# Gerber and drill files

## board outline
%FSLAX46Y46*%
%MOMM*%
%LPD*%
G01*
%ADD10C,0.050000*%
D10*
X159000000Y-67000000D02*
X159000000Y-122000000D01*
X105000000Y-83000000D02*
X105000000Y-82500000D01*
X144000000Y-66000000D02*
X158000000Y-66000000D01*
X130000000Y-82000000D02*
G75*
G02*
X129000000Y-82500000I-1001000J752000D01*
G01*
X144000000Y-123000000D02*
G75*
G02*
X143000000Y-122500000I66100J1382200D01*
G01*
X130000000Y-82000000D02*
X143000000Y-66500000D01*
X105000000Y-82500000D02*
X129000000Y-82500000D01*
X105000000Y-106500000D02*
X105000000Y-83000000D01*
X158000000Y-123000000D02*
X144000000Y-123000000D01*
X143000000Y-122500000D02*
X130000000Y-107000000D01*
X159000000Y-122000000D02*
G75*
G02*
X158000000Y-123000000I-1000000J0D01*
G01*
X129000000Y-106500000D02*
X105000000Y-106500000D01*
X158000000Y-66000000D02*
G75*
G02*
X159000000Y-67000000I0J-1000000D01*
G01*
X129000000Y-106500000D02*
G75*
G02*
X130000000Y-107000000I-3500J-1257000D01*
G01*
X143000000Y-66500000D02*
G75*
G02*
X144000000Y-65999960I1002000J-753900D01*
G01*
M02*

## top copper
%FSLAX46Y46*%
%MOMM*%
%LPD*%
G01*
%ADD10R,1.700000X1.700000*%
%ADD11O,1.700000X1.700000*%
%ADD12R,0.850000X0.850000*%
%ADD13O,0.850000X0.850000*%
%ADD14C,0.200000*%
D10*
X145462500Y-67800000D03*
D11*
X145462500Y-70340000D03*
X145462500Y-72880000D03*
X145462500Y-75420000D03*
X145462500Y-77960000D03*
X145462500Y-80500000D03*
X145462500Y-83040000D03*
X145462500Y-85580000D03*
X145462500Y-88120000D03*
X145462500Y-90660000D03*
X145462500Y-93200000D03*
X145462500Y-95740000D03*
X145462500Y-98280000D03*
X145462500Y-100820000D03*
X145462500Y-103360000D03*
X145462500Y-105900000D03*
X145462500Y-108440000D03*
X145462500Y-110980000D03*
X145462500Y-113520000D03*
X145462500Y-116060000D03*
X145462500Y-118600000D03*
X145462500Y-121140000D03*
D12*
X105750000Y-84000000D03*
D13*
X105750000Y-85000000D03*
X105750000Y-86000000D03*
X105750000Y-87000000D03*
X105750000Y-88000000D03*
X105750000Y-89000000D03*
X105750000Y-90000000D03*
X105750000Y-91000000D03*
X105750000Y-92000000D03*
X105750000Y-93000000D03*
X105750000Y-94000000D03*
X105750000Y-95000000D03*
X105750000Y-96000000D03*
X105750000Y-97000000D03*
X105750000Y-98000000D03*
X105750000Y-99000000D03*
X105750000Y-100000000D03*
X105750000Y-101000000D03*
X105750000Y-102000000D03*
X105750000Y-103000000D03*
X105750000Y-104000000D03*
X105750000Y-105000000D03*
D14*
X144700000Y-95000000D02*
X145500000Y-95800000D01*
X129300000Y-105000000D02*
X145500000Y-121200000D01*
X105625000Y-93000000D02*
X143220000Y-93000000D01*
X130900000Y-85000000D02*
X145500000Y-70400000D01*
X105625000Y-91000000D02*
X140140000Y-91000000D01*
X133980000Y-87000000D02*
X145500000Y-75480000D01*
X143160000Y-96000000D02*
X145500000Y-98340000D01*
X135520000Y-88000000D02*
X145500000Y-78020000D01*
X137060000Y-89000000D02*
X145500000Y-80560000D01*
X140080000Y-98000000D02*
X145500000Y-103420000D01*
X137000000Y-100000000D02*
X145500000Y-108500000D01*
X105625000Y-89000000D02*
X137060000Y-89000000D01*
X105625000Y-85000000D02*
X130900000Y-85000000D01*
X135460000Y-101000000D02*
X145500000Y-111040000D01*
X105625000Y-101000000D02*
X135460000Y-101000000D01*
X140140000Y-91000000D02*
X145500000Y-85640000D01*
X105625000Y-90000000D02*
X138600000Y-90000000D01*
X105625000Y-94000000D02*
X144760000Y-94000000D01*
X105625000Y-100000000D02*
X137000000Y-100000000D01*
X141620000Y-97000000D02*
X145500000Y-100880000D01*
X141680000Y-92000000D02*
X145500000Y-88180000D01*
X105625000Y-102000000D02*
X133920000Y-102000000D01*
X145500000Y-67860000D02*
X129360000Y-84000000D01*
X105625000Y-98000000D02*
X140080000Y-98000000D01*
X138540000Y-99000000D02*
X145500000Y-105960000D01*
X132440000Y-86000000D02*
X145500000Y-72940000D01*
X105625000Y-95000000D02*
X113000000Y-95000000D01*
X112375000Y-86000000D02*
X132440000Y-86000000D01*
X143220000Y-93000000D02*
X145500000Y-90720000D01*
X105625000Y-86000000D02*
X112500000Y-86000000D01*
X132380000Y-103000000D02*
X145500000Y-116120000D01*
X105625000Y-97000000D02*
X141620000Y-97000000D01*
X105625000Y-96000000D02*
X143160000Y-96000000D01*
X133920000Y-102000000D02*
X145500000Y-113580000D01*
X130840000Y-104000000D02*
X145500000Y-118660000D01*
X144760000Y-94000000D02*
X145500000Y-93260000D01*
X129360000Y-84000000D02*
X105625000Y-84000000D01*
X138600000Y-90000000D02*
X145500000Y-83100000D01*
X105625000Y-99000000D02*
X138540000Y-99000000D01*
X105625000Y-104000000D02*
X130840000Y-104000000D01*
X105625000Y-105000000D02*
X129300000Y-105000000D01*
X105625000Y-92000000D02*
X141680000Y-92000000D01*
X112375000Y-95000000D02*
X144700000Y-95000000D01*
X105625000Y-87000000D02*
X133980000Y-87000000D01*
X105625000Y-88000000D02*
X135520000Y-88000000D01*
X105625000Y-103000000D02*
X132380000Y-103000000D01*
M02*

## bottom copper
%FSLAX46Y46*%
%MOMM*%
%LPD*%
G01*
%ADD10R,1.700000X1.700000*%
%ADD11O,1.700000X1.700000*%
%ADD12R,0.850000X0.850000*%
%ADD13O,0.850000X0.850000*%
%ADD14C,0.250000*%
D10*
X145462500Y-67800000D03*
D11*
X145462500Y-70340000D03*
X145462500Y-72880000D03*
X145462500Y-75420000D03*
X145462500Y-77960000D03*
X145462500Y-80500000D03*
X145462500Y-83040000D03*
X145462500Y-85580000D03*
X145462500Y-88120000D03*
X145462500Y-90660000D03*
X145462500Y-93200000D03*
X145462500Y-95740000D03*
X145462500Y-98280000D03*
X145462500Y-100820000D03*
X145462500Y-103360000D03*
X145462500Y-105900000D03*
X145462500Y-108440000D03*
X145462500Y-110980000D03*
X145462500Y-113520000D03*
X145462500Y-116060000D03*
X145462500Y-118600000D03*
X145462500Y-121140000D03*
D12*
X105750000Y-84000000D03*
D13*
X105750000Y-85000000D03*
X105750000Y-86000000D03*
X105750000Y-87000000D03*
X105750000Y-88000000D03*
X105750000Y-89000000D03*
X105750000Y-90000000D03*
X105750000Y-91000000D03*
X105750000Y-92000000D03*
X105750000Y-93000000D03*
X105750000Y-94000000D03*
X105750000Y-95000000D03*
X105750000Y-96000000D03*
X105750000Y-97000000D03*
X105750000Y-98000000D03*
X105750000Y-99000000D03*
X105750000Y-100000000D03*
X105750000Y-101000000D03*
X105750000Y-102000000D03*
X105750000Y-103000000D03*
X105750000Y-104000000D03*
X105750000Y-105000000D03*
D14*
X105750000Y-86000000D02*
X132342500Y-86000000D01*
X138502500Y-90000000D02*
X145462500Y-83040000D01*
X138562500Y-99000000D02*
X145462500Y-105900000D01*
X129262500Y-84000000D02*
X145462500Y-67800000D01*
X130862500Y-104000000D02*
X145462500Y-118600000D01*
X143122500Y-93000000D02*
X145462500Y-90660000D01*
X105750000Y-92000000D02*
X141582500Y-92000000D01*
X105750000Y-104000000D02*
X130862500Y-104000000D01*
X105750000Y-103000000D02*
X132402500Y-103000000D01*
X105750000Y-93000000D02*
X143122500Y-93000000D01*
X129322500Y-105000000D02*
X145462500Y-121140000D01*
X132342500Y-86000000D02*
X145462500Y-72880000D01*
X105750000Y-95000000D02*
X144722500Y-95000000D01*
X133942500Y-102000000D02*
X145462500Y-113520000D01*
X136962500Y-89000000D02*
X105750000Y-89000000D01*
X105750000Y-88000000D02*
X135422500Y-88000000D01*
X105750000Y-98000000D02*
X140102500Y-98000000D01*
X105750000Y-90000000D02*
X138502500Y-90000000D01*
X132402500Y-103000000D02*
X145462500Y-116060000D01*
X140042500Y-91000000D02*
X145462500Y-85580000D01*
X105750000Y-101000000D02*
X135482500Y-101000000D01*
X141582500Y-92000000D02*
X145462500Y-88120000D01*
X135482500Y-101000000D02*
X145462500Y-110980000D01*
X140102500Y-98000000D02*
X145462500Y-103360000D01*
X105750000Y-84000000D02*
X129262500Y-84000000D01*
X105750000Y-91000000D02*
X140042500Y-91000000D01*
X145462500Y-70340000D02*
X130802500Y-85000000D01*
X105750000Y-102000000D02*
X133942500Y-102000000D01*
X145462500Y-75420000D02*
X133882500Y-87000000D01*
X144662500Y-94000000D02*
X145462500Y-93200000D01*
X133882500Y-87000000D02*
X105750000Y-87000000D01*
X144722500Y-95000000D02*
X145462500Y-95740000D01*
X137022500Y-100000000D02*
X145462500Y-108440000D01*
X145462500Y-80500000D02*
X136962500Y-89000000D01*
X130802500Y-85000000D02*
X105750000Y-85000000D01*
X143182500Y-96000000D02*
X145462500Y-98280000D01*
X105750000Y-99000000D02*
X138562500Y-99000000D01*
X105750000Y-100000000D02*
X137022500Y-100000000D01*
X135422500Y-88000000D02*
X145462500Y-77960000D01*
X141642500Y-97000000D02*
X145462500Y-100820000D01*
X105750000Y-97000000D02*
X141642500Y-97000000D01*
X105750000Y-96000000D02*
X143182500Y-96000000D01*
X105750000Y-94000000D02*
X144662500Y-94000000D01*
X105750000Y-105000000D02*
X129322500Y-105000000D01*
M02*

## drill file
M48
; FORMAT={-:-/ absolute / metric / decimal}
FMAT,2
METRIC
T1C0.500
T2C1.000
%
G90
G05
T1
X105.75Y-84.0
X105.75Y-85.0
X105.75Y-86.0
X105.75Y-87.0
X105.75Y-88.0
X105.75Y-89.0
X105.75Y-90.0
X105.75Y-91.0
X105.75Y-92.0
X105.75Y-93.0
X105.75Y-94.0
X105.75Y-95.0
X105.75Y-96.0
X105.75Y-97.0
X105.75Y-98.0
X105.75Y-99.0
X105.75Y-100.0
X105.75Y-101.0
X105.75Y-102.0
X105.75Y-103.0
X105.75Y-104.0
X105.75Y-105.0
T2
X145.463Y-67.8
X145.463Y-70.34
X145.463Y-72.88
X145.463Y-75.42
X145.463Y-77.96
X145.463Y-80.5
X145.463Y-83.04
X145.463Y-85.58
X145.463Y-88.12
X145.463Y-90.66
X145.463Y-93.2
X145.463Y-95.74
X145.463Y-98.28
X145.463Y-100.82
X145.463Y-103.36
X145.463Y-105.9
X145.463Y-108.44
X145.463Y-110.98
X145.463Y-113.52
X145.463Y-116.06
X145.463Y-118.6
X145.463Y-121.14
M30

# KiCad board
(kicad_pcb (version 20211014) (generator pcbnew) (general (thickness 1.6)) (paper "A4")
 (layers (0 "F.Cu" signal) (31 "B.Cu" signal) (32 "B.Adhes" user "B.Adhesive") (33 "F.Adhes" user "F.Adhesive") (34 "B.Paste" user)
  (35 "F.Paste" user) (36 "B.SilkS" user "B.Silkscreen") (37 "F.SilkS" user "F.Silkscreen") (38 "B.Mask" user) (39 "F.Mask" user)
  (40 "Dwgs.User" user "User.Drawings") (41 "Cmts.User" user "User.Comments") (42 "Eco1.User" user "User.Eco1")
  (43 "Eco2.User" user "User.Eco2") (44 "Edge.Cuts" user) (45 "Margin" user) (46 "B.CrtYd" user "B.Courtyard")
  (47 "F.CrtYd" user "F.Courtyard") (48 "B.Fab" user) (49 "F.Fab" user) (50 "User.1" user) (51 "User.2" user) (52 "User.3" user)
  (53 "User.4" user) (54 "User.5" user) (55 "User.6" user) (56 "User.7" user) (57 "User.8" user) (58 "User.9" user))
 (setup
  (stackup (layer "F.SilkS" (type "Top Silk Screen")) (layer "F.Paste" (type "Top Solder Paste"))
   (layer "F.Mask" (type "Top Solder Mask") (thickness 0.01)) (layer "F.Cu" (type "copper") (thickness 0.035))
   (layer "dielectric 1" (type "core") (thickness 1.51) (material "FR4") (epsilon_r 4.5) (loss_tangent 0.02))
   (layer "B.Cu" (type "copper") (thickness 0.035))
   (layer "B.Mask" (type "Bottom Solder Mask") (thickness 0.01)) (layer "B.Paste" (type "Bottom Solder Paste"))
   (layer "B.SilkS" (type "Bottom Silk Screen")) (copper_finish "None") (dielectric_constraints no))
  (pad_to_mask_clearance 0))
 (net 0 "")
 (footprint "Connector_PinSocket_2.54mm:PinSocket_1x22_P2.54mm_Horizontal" (layer "F.Cu") (at 159.0625 67.8)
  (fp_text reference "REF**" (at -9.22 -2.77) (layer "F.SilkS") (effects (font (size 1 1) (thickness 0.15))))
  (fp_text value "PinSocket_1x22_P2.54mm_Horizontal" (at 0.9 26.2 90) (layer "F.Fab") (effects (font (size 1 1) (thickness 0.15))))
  (pad "1" thru_hole rect (at -13.6 0) (size 1.7 1.7) (drill 1) (layers *.Cu *.Mask))
  (pad "2" thru_hole oval (at -13.6 2.54) (size 1.7 1.7) (drill 1) (layers *.Cu *.Mask))
  (pad "3" thru_hole oval (at -13.6 5.08) (size 1.7 1.7) (drill 1) (layers *.Cu *.Mask))
  (pad "4" thru_hole oval (at -13.6 7.62) (size 1.7 1.7) (drill 1) (layers *.Cu *.Mask))
  (pad "5" thru_hole oval (at -13.6 10.16) (size 1.7 1.7) (drill 1) (layers *.Cu *.Mask))
  (pad "6" thru_hole oval (at -13.6 12.7) (size 1.7 1.7) (drill 1) (layers *.Cu *.Mask))
  (pad "7" thru_hole oval (at -13.6 15.24) (size 1.7 1.7) (drill 1) (layers *.Cu *.Mask))
  (pad "8" thru_hole oval (at -13.6 17.78) (size 1.7 1.7) (drill 1) (layers *.Cu *.Mask))
  (pad "9" thru_hole oval (at -13.6 20.32) (size 1.7 1.7) (drill 1) (layers *.Cu *.Mask))
  (pad "10" thru_hole oval (at -13.6 22.86) (size 1.7 1.7) (drill 1) (layers *.Cu *.Mask))
  (pad "11" thru_hole oval (at -13.6 25.4) (size 1.7 1.7) (drill 1) (layers *.Cu *.Mask))
  (pad "12" thru_hole oval (at -13.6 27.94) (size 1.7 1.7) (drill 1) (layers *.Cu *.Mask))
  (pad "13" thru_hole oval (at -13.6 30.48) (size 1.7 1.7) (drill 1) (layers *.Cu *.Mask))
  (pad "14" thru_hole oval (at -13.6 33.02) (size 1.7 1.7) (drill 1) (layers *.Cu *.Mask))
  (pad "15" thru_hole oval (at -13.6 35.56) (size 1.7 1.7) (drill 1) (layers *.Cu *.Mask))
  (pad "16" thru_hole oval (at -13.6 38.1) (size 1.7 1.7) (drill 1) (layers *.Cu *.Mask))
  (pad "17" thru_hole oval (at -13.6 40.64) (size 1.7 1.7) (drill 1) (layers *.Cu *.Mask))
  (pad "18" thru_hole oval (at -13.6 43.18) (size 1.7 1.7) (drill 1) (layers *.Cu *.Mask))
  (pad "19" thru_hole oval (at -13.6 45.72) (size 1.7 1.7) (drill 1) (layers *.Cu *.Mask))
  (pad "20" thru_hole oval (at -13.6 48.26) (size 1.7 1.7) (drill 1) (layers *.Cu *.Mask))
  (pad "21" thru_hole oval (at -13.6 50.8) (size 1.7 1.7) (drill 1) (layers *.Cu *.Mask))
  (pad "22" thru_hole oval (at -13.6 53.34) (size 1.7 1.7) (drill 1) (layers *.Cu *.Mask)))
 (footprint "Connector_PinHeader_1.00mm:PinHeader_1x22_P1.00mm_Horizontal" (layer "F.Cu") (at 100.15 84)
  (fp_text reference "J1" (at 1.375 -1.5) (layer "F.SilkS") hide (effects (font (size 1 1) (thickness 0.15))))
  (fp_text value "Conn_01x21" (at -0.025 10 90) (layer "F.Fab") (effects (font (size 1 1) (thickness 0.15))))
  (pad "1" thru_hole rect (at 5.6 0) (size 0.85 0.85) (drill 0.5) (layers *.Cu *.Mask))
  (pad "2" thru_hole oval (at 5.6 1) (size 0.85 0.85) (drill 0.5) (layers *.Cu *.Mask))
  (pad "3" thru_hole oval (at 5.6 2) (size 0.85 0.85) (drill 0.5) (layers *.Cu *.Mask))
  (pad "4" thru_hole oval (at 5.6 3) (size 0.85 0.85) (drill 0.5) (layers *.Cu *.Mask))
  (pad "5" thru_hole oval (at 5.6 4) (size 0.85 0.85) (drill 0.5) (layers *.Cu *.Mask))
  (pad "6" thru_hole oval (at 5.6 5) (size 0.85 0.85) (drill 0.5) (layers *.Cu *.Mask))
  (pad "7" thru_hole oval (at 5.6 6) (size 0.85 0.85) (drill 0.5) (layers *.Cu *.Mask))
  (pad "8" thru_hole oval (at 5.6 7) (size 0.85 0.85) (drill 0.5) (layers *.Cu *.Mask))
  (pad "9" thru_hole oval (at 5.6 8) (size 0.85 0.85) (drill 0.5) (layers *.Cu *.Mask))
  (pad "10" thru_hole oval (at 5.6 9) (size 0.85 0.85) (drill 0.5) (layers *.Cu *.Mask))
  (pad "11" thru_hole oval (at 5.6 10) (size 0.85 0.85) (drill 0.5) (layers *.Cu *.Mask))
  (pad "12" thru_hole oval (at 5.6 11) (size 0.85 0.85) (drill 0.5) (layers *.Cu *.Mask))
  (pad "13" thru_hole oval (at 5.6 12) (size 0.85 0.85) (drill 0.5) (layers *.Cu *.Mask))
  (pad "14" thru_hole oval (at 5.6 13) (size 0.85 0.85) (drill 0.5) (layers *.Cu *.Mask))
  (pad "15" thru_hole oval (at 5.6 14) (size 0.85 0.85) (drill 0.5) (layers *.Cu *.Mask))
  (pad "16" thru_hole oval (at 5.6 15) (size 0.85 0.85) (drill 0.5) (layers *.Cu *.Mask))
  (pad "17" thru_hole oval (at 5.6 16) (size 0.85 0.85) (drill 0.5) (layers *.Cu *.Mask))
  (pad "18" thru_hole oval (at 5.6 17) (size 0.85 0.85) (drill 0.5) (layers *.Cu *.Mask))
  (pad "19" thru_hole oval (at 5.6 18) (size 0.85 0.85) (drill 0.5) (layers *.Cu *.Mask))
  (pad "20" thru_hole oval (at 5.6 19) (size 0.85 0.85) (drill 0.5) (layers *.Cu *.Mask))
  (pad "21" thru_hole oval (at 5.6 20) (size 0.85 0.85) (drill 0.5) (layers *.Cu *.Mask))
  (pad "22" thru_hole oval (at 5.6 21) (size 0.85 0.85) (drill 0.5) (layers *.Cu *.Mask)))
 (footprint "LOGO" (layer "F.Cu") (at 135.15 84.3 90)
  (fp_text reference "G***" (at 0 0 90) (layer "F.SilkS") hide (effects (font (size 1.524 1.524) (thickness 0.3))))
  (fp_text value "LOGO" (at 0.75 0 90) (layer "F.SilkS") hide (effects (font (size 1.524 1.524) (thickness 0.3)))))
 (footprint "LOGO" (layer "B.Cu") (at 135.119123 104.632972 -90)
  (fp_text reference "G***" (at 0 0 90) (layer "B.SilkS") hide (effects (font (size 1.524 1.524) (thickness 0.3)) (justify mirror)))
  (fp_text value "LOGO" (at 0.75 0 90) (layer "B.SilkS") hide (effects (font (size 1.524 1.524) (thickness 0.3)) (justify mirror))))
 (gr_line (start 159 67) (end 159 122) (layer "Edge.Cuts") (width 0.05))
 (gr_line (start 105 83) (end 105 82.5) (layer "Edge.Cuts") (width 0.05))
 (gr_line (start 144 66) (end 158 66) (layer "Edge.Cuts") (width 0.05))
 (gr_arc (start 130 82) (mid 129.558911 82.367822) (end 129 82.5) (layer "Edge.Cuts") (width 0.05))
 (gr_arc (start 144 123) (mid 143.447254 122.855491) (end 143 122.5) (layer "Edge.Cuts") (width 0.05))
 (gr_line (start 130 82) (end 143 66.5) (layer "Edge.Cuts") (width 0.05))
 (gr_line (start 105 82.5) (end 129 82.5) (layer "Edge.Cuts") (width 0.05))
 (gr_line (start 105 106.5) (end 105 83) (layer "Edge.Cuts") (width 0.05))
 (gr_line (start 158 123) (end 144 123) (layer "Edge.Cuts") (width 0.05))
 (gr_line (start 143 122.5) (end 130 107) (layer "Edge.Cuts") (width 0.05))
 (gr_arc (start 159 122) (mid 158.707107 122.707107) (end 158 123) (layer "Edge.Cuts") (width 0.05))
 (gr_line (start 129 106.5) (end 105 106.5) (layer "Edge.Cuts") (width 0.05))
 (gr_arc (start 158 66) (mid 158.707107 66.292893) (end 159 67) (layer "Edge.Cuts") (width 0.05))
 (gr_arc (start 129 106.5) (mid 129.558648 106.632703) (end 130 107) (layer "Edge.Cuts") (width 0.05))
 (gr_arc (start 143 66.5) (mid 143.44119 66.132381) (end 144 66) (layer "Edge.Cuts") (width 0.05))
 (segment (start 144.7 95) (end 145.5 95.8) (width 0.2) (layer "F.Cu") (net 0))
 (segment (start 129.3 105) (end 145.5 121.2) (width 0.2) (layer "F.Cu") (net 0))
 (segment (start 105.625 93) (end 143.22 93) (width 0.2) (layer "F.Cu") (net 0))
 (segment (start 130.9 85) (end 145.5 70.4) (width 0.2) (layer "F.Cu") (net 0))
 (segment (start 105.625 91) (end 140.14 91) (width 0.2) (layer "F.Cu") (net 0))
 (segment (start 133.98 87) (end 145.5 75.48) (width 0.2) (layer "F.Cu") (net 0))
 (segment (start 143.16 96) (end 145.5 98.34) (width 0.2) (layer "F.Cu") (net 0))
 (segment (start 135.52 88) (end 145.5 78.02) (width 0.2) (layer "F.Cu") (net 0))
 (segment (start 137.06 89) (end 145.5 80.56) (width 0.2) (layer "F.Cu") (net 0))
 (segment (start 140.08 98) (end 145.5 103.42) (width 0.2) (layer "F.Cu") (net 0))
 (segment (start 137 100) (end 145.5 108.5) (width 0.2) (layer "F.Cu") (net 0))
 (segment (start 105.625 89) (end 137.06 89) (width 0.2) (layer "F.Cu") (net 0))
 (segment (start 105.625 85) (end 130.9 85) (width 0.2) (layer "F.Cu") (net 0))
 (segment (start 135.46 101) (end 145.5 111.04) (width 0.2) (layer "F.Cu") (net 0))
 (segment (start 105.625 101) (end 135.46 101) (width 0.2) (layer "F.Cu") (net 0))
 (segment (start 140.14 91) (end 145.5 85.64) (width 0.2) (layer "F.Cu") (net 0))
 (segment (start 105.625 90) (end 138.6 90) (width 0.2) (layer "F.Cu") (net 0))
 (segment (start 105.625 94) (end 144.76 94) (width 0.2) (layer "F.Cu") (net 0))
 (segment (start 105.625 100) (end 137 100) (width 0.2) (layer "F.Cu") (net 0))
 (segment (start 141.62 97) (end 145.5 100.88) (width 0.2) (layer "F.Cu") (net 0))
 (segment (start 141.68 92) (end 145.5 88.18) (width 0.2) (layer "F.Cu") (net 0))
 (segment (start 105.625 102) (end 133.92 102) (width 0.2) (layer "F.Cu") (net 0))
 (segment (start 145.5 67.86) (end 129.36 84) (width 0.2) (layer "F.Cu") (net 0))
 (segment (start 105.625 98) (end 140.08 98) (width 0.2) (layer "F.Cu") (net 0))
 (segment (start 138.54 99) (end 145.5 105.96) (width 0.2) (layer "F.Cu") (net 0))
 (segment (start 132.44 86) (end 145.5 72.94) (width 0.2) (layer "F.Cu") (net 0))
 (segment (start 105.625 95) (end 113 95) (width 0.2) (layer "F.Cu") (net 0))
 (segment (start 112.375 86) (end 132.44 86) (width 0.2) (layer "F.Cu") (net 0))
 (segment (start 143.22 93) (end 145.5 90.72) (width 0.2) (layer "F.Cu") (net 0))
 (segment (start 105.625 86) (end 112.5 86) (width 0.2) (layer "F.Cu") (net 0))
 (segment (start 132.38 103) (end 145.5 116.12) (width 0.2) (layer "F.Cu") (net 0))
 (segment (start 105.625 97) (end 141.62 97) (width 0.2) (layer "F.Cu") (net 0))
 (segment (start 105.625 96) (end 143.16 96) (width 0.2) (layer "F.Cu") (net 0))
 (segment (start 133.92 102) (end 145.5 113.58) (width 0.2) (layer "F.Cu") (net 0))
 (segment (start 130.84 104) (end 145.5 118.66) (width 0.2) (layer "F.Cu") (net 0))
 (segment (start 144.76 94) (end 145.5 93.26) (width 0.2) (layer "F.Cu") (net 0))
 (segment (start 129.36 84) (end 105.625 84) (width 0.2) (layer "F.Cu") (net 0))
 (segment (start 138.6 90) (end 145.5 83.1) (width 0.2) (layer "F.Cu") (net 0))
 (segment (start 105.625 99) (end 138.54 99) (width 0.2) (layer "F.Cu") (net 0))
 (segment (start 105.625 104) (end 130.84 104) (width 0.2) (layer "F.Cu") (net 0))
 (segment (start 105.625 105) (end 129.3 105) (width 0.2) (layer "F.Cu") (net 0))
 (segment (start 105.625 92) (end 141.68 92) (width 0.2) (layer "F.Cu") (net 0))
 (segment (start 112.375 95) (end 144.7 95) (width 0.2) (layer "F.Cu") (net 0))
 (segment (start 105.625 87) (end 133.98 87) (width 0.2) (layer "F.Cu") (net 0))
 (segment (start 105.625 88) (end 135.52 88) (width 0.2) (layer "F.Cu") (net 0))
 (segment (start 105.625 103) (end 132.38 103) (width 0.2) (layer "F.Cu") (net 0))
 (segment (start 105.75 86) (end 132.3425 86) (width 0.25) (layer "B.Cu") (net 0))
 (segment (start 138.5025 90) (end 145.4625 83.04) (width 0.25) (layer "B.Cu") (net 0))
 (segment (start 138.5625 99) (end 145.4625 105.9) (width 0.25) (layer "B.Cu") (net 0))
 (segment (start 129.2625 84) (end 145.4625 67.8) (width 0.25) (layer "B.Cu") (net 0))
 (segment (start 130.8625 104) (end 145.4625 118.6) (width 0.25) (layer "B.Cu") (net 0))
 (segment (start 143.1225 93) (end 145.4625 90.66) (width 0.25) (layer "B.Cu") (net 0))
 (segment (start 105.75 92) (end 141.5825 92) (width 0.25) (layer "B.Cu") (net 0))
 (segment (start 105.75 104) (end 130.8625 104) (width 0.25) (layer "B.Cu") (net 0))
 (segment (start 105.75 103) (end 132.4025 103) (width 0.25) (layer "B.Cu") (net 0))
 (segment (start 105.75 93) (end 143.1225 93) (width 0.25) (layer "B.Cu") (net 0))
 (segment (start 129.3225 105) (end 145.4625 121.14) (width 0.25) (layer "B.Cu") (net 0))
 (segment (start 132.3425 86) (end 145.4625 72.88) (width 0.25) (layer "B.Cu") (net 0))
 (segment (start 105.75 95) (end 144.7225 95) (width 0.25) (layer "B.Cu") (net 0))
 (segment (start 133.9425 102) (end 145.4625 113.52) (width 0.25) (layer "B.Cu") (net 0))
 (segment (start 136.9625 89) (end 105.75 89) (width 0.25) (layer "B.Cu") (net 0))
 (segment (start 105.75 88) (end 135.4225 88) (width 0.25) (layer "B.Cu") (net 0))
 (segment (start 105.75 98) (end 140.1025 98) (width 0.25) (layer "B.Cu") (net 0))
 (segment (start 105.75 90) (end 138.5025 90) (width 0.25) (layer "B.Cu") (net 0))
 (segment (start 132.4025 103) (end 145.4625 116.06) (width 0.25) (layer "B.Cu") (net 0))
 (segment (start 140.0425 91) (end 145.4625 85.58) (width 0.25) (layer "B.Cu") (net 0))
 (segment (start 105.75 101) (end 135.4825 101) (width 0.25) (layer "B.Cu") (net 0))
 (segment (start 141.5825 92) (end 145.4625 88.12) (width 0.25) (layer "B.Cu") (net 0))
 (segment (start 135.4825 101) (end 145.4625 110.98) (width 0.25) (layer "B.Cu") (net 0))
 (segment (start 140.1025 98) (end 145.4625 103.36) (width 0.25) (layer "B.Cu") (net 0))
 (segment (start 105.75 84) (end 129.2625 84) (width 0.25) (layer "B.Cu") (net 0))
 (segment (start 105.75 91) (end 140.0425 91) (width 0.25) (layer "B.Cu") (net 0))
 (segment (start 145.4625 70.34) (end 130.8025 85) (width 0.25) (layer "B.Cu") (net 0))
 (segment (start 105.75 102) (end 133.9425 102) (width 0.25) (layer "B.Cu") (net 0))
 (segment (start 145.4625 75.42) (end 133.8825 87) (width 0.25) (layer "B.Cu") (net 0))
 (segment (start 144.6625 94) (end 145.4625 93.2) (width 0.25) (layer "B.Cu") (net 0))
 (segment (start 133.8825 87) (end 105.75 87) (width 0.25) (layer "B.Cu") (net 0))
 (segment (start 144.7225 95) (end 145.4625 95.74) (width 0.25) (layer "B.Cu") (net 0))
 (segment (start 137.0225 100) (end 145.4625 108.44) (width 0.25) (layer "B.Cu") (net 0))
 (segment (start 145.4625 80.5) (end 136.9625 89) (width 0.25) (layer "B.Cu") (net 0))
 (segment (start 130.8025 85) (end 105.75 85) (width 0.25) (layer "B.Cu") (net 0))
 (segment (start 143.1825 96) (end 145.4625 98.28) (width 0.25) (layer "B.Cu") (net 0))
 (segment (start 105.75 99) (end 138.5625 99) (width 0.25) (layer "B.Cu") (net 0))
 (segment (start 105.75 100) (end 137.0225 100) (width 0.25) (layer "B.Cu") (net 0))
 (segment (start 135.4225 88) (end 145.4625 77.96) (width 0.25) (layer "B.Cu") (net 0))
 (segment (start 141.6425 97) (end 145.4625 100.82) (width 0.25) (layer "B.Cu") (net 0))
 (segment (start 105.75 97) (end 141.6425 97) (width 0.25) (layer "B.Cu") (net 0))
 (segment (start 105.75 96) (end 143.1825 96) (width 0.25) (layer "B.Cu") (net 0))
 (segment (start 105.75 94) (end 144.6625 94) (width 0.25) (layer "B.Cu") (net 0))
 (segment (start 105.75 105) (end 129.3225 105) (width 0.25) (layer "B.Cu") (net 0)))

